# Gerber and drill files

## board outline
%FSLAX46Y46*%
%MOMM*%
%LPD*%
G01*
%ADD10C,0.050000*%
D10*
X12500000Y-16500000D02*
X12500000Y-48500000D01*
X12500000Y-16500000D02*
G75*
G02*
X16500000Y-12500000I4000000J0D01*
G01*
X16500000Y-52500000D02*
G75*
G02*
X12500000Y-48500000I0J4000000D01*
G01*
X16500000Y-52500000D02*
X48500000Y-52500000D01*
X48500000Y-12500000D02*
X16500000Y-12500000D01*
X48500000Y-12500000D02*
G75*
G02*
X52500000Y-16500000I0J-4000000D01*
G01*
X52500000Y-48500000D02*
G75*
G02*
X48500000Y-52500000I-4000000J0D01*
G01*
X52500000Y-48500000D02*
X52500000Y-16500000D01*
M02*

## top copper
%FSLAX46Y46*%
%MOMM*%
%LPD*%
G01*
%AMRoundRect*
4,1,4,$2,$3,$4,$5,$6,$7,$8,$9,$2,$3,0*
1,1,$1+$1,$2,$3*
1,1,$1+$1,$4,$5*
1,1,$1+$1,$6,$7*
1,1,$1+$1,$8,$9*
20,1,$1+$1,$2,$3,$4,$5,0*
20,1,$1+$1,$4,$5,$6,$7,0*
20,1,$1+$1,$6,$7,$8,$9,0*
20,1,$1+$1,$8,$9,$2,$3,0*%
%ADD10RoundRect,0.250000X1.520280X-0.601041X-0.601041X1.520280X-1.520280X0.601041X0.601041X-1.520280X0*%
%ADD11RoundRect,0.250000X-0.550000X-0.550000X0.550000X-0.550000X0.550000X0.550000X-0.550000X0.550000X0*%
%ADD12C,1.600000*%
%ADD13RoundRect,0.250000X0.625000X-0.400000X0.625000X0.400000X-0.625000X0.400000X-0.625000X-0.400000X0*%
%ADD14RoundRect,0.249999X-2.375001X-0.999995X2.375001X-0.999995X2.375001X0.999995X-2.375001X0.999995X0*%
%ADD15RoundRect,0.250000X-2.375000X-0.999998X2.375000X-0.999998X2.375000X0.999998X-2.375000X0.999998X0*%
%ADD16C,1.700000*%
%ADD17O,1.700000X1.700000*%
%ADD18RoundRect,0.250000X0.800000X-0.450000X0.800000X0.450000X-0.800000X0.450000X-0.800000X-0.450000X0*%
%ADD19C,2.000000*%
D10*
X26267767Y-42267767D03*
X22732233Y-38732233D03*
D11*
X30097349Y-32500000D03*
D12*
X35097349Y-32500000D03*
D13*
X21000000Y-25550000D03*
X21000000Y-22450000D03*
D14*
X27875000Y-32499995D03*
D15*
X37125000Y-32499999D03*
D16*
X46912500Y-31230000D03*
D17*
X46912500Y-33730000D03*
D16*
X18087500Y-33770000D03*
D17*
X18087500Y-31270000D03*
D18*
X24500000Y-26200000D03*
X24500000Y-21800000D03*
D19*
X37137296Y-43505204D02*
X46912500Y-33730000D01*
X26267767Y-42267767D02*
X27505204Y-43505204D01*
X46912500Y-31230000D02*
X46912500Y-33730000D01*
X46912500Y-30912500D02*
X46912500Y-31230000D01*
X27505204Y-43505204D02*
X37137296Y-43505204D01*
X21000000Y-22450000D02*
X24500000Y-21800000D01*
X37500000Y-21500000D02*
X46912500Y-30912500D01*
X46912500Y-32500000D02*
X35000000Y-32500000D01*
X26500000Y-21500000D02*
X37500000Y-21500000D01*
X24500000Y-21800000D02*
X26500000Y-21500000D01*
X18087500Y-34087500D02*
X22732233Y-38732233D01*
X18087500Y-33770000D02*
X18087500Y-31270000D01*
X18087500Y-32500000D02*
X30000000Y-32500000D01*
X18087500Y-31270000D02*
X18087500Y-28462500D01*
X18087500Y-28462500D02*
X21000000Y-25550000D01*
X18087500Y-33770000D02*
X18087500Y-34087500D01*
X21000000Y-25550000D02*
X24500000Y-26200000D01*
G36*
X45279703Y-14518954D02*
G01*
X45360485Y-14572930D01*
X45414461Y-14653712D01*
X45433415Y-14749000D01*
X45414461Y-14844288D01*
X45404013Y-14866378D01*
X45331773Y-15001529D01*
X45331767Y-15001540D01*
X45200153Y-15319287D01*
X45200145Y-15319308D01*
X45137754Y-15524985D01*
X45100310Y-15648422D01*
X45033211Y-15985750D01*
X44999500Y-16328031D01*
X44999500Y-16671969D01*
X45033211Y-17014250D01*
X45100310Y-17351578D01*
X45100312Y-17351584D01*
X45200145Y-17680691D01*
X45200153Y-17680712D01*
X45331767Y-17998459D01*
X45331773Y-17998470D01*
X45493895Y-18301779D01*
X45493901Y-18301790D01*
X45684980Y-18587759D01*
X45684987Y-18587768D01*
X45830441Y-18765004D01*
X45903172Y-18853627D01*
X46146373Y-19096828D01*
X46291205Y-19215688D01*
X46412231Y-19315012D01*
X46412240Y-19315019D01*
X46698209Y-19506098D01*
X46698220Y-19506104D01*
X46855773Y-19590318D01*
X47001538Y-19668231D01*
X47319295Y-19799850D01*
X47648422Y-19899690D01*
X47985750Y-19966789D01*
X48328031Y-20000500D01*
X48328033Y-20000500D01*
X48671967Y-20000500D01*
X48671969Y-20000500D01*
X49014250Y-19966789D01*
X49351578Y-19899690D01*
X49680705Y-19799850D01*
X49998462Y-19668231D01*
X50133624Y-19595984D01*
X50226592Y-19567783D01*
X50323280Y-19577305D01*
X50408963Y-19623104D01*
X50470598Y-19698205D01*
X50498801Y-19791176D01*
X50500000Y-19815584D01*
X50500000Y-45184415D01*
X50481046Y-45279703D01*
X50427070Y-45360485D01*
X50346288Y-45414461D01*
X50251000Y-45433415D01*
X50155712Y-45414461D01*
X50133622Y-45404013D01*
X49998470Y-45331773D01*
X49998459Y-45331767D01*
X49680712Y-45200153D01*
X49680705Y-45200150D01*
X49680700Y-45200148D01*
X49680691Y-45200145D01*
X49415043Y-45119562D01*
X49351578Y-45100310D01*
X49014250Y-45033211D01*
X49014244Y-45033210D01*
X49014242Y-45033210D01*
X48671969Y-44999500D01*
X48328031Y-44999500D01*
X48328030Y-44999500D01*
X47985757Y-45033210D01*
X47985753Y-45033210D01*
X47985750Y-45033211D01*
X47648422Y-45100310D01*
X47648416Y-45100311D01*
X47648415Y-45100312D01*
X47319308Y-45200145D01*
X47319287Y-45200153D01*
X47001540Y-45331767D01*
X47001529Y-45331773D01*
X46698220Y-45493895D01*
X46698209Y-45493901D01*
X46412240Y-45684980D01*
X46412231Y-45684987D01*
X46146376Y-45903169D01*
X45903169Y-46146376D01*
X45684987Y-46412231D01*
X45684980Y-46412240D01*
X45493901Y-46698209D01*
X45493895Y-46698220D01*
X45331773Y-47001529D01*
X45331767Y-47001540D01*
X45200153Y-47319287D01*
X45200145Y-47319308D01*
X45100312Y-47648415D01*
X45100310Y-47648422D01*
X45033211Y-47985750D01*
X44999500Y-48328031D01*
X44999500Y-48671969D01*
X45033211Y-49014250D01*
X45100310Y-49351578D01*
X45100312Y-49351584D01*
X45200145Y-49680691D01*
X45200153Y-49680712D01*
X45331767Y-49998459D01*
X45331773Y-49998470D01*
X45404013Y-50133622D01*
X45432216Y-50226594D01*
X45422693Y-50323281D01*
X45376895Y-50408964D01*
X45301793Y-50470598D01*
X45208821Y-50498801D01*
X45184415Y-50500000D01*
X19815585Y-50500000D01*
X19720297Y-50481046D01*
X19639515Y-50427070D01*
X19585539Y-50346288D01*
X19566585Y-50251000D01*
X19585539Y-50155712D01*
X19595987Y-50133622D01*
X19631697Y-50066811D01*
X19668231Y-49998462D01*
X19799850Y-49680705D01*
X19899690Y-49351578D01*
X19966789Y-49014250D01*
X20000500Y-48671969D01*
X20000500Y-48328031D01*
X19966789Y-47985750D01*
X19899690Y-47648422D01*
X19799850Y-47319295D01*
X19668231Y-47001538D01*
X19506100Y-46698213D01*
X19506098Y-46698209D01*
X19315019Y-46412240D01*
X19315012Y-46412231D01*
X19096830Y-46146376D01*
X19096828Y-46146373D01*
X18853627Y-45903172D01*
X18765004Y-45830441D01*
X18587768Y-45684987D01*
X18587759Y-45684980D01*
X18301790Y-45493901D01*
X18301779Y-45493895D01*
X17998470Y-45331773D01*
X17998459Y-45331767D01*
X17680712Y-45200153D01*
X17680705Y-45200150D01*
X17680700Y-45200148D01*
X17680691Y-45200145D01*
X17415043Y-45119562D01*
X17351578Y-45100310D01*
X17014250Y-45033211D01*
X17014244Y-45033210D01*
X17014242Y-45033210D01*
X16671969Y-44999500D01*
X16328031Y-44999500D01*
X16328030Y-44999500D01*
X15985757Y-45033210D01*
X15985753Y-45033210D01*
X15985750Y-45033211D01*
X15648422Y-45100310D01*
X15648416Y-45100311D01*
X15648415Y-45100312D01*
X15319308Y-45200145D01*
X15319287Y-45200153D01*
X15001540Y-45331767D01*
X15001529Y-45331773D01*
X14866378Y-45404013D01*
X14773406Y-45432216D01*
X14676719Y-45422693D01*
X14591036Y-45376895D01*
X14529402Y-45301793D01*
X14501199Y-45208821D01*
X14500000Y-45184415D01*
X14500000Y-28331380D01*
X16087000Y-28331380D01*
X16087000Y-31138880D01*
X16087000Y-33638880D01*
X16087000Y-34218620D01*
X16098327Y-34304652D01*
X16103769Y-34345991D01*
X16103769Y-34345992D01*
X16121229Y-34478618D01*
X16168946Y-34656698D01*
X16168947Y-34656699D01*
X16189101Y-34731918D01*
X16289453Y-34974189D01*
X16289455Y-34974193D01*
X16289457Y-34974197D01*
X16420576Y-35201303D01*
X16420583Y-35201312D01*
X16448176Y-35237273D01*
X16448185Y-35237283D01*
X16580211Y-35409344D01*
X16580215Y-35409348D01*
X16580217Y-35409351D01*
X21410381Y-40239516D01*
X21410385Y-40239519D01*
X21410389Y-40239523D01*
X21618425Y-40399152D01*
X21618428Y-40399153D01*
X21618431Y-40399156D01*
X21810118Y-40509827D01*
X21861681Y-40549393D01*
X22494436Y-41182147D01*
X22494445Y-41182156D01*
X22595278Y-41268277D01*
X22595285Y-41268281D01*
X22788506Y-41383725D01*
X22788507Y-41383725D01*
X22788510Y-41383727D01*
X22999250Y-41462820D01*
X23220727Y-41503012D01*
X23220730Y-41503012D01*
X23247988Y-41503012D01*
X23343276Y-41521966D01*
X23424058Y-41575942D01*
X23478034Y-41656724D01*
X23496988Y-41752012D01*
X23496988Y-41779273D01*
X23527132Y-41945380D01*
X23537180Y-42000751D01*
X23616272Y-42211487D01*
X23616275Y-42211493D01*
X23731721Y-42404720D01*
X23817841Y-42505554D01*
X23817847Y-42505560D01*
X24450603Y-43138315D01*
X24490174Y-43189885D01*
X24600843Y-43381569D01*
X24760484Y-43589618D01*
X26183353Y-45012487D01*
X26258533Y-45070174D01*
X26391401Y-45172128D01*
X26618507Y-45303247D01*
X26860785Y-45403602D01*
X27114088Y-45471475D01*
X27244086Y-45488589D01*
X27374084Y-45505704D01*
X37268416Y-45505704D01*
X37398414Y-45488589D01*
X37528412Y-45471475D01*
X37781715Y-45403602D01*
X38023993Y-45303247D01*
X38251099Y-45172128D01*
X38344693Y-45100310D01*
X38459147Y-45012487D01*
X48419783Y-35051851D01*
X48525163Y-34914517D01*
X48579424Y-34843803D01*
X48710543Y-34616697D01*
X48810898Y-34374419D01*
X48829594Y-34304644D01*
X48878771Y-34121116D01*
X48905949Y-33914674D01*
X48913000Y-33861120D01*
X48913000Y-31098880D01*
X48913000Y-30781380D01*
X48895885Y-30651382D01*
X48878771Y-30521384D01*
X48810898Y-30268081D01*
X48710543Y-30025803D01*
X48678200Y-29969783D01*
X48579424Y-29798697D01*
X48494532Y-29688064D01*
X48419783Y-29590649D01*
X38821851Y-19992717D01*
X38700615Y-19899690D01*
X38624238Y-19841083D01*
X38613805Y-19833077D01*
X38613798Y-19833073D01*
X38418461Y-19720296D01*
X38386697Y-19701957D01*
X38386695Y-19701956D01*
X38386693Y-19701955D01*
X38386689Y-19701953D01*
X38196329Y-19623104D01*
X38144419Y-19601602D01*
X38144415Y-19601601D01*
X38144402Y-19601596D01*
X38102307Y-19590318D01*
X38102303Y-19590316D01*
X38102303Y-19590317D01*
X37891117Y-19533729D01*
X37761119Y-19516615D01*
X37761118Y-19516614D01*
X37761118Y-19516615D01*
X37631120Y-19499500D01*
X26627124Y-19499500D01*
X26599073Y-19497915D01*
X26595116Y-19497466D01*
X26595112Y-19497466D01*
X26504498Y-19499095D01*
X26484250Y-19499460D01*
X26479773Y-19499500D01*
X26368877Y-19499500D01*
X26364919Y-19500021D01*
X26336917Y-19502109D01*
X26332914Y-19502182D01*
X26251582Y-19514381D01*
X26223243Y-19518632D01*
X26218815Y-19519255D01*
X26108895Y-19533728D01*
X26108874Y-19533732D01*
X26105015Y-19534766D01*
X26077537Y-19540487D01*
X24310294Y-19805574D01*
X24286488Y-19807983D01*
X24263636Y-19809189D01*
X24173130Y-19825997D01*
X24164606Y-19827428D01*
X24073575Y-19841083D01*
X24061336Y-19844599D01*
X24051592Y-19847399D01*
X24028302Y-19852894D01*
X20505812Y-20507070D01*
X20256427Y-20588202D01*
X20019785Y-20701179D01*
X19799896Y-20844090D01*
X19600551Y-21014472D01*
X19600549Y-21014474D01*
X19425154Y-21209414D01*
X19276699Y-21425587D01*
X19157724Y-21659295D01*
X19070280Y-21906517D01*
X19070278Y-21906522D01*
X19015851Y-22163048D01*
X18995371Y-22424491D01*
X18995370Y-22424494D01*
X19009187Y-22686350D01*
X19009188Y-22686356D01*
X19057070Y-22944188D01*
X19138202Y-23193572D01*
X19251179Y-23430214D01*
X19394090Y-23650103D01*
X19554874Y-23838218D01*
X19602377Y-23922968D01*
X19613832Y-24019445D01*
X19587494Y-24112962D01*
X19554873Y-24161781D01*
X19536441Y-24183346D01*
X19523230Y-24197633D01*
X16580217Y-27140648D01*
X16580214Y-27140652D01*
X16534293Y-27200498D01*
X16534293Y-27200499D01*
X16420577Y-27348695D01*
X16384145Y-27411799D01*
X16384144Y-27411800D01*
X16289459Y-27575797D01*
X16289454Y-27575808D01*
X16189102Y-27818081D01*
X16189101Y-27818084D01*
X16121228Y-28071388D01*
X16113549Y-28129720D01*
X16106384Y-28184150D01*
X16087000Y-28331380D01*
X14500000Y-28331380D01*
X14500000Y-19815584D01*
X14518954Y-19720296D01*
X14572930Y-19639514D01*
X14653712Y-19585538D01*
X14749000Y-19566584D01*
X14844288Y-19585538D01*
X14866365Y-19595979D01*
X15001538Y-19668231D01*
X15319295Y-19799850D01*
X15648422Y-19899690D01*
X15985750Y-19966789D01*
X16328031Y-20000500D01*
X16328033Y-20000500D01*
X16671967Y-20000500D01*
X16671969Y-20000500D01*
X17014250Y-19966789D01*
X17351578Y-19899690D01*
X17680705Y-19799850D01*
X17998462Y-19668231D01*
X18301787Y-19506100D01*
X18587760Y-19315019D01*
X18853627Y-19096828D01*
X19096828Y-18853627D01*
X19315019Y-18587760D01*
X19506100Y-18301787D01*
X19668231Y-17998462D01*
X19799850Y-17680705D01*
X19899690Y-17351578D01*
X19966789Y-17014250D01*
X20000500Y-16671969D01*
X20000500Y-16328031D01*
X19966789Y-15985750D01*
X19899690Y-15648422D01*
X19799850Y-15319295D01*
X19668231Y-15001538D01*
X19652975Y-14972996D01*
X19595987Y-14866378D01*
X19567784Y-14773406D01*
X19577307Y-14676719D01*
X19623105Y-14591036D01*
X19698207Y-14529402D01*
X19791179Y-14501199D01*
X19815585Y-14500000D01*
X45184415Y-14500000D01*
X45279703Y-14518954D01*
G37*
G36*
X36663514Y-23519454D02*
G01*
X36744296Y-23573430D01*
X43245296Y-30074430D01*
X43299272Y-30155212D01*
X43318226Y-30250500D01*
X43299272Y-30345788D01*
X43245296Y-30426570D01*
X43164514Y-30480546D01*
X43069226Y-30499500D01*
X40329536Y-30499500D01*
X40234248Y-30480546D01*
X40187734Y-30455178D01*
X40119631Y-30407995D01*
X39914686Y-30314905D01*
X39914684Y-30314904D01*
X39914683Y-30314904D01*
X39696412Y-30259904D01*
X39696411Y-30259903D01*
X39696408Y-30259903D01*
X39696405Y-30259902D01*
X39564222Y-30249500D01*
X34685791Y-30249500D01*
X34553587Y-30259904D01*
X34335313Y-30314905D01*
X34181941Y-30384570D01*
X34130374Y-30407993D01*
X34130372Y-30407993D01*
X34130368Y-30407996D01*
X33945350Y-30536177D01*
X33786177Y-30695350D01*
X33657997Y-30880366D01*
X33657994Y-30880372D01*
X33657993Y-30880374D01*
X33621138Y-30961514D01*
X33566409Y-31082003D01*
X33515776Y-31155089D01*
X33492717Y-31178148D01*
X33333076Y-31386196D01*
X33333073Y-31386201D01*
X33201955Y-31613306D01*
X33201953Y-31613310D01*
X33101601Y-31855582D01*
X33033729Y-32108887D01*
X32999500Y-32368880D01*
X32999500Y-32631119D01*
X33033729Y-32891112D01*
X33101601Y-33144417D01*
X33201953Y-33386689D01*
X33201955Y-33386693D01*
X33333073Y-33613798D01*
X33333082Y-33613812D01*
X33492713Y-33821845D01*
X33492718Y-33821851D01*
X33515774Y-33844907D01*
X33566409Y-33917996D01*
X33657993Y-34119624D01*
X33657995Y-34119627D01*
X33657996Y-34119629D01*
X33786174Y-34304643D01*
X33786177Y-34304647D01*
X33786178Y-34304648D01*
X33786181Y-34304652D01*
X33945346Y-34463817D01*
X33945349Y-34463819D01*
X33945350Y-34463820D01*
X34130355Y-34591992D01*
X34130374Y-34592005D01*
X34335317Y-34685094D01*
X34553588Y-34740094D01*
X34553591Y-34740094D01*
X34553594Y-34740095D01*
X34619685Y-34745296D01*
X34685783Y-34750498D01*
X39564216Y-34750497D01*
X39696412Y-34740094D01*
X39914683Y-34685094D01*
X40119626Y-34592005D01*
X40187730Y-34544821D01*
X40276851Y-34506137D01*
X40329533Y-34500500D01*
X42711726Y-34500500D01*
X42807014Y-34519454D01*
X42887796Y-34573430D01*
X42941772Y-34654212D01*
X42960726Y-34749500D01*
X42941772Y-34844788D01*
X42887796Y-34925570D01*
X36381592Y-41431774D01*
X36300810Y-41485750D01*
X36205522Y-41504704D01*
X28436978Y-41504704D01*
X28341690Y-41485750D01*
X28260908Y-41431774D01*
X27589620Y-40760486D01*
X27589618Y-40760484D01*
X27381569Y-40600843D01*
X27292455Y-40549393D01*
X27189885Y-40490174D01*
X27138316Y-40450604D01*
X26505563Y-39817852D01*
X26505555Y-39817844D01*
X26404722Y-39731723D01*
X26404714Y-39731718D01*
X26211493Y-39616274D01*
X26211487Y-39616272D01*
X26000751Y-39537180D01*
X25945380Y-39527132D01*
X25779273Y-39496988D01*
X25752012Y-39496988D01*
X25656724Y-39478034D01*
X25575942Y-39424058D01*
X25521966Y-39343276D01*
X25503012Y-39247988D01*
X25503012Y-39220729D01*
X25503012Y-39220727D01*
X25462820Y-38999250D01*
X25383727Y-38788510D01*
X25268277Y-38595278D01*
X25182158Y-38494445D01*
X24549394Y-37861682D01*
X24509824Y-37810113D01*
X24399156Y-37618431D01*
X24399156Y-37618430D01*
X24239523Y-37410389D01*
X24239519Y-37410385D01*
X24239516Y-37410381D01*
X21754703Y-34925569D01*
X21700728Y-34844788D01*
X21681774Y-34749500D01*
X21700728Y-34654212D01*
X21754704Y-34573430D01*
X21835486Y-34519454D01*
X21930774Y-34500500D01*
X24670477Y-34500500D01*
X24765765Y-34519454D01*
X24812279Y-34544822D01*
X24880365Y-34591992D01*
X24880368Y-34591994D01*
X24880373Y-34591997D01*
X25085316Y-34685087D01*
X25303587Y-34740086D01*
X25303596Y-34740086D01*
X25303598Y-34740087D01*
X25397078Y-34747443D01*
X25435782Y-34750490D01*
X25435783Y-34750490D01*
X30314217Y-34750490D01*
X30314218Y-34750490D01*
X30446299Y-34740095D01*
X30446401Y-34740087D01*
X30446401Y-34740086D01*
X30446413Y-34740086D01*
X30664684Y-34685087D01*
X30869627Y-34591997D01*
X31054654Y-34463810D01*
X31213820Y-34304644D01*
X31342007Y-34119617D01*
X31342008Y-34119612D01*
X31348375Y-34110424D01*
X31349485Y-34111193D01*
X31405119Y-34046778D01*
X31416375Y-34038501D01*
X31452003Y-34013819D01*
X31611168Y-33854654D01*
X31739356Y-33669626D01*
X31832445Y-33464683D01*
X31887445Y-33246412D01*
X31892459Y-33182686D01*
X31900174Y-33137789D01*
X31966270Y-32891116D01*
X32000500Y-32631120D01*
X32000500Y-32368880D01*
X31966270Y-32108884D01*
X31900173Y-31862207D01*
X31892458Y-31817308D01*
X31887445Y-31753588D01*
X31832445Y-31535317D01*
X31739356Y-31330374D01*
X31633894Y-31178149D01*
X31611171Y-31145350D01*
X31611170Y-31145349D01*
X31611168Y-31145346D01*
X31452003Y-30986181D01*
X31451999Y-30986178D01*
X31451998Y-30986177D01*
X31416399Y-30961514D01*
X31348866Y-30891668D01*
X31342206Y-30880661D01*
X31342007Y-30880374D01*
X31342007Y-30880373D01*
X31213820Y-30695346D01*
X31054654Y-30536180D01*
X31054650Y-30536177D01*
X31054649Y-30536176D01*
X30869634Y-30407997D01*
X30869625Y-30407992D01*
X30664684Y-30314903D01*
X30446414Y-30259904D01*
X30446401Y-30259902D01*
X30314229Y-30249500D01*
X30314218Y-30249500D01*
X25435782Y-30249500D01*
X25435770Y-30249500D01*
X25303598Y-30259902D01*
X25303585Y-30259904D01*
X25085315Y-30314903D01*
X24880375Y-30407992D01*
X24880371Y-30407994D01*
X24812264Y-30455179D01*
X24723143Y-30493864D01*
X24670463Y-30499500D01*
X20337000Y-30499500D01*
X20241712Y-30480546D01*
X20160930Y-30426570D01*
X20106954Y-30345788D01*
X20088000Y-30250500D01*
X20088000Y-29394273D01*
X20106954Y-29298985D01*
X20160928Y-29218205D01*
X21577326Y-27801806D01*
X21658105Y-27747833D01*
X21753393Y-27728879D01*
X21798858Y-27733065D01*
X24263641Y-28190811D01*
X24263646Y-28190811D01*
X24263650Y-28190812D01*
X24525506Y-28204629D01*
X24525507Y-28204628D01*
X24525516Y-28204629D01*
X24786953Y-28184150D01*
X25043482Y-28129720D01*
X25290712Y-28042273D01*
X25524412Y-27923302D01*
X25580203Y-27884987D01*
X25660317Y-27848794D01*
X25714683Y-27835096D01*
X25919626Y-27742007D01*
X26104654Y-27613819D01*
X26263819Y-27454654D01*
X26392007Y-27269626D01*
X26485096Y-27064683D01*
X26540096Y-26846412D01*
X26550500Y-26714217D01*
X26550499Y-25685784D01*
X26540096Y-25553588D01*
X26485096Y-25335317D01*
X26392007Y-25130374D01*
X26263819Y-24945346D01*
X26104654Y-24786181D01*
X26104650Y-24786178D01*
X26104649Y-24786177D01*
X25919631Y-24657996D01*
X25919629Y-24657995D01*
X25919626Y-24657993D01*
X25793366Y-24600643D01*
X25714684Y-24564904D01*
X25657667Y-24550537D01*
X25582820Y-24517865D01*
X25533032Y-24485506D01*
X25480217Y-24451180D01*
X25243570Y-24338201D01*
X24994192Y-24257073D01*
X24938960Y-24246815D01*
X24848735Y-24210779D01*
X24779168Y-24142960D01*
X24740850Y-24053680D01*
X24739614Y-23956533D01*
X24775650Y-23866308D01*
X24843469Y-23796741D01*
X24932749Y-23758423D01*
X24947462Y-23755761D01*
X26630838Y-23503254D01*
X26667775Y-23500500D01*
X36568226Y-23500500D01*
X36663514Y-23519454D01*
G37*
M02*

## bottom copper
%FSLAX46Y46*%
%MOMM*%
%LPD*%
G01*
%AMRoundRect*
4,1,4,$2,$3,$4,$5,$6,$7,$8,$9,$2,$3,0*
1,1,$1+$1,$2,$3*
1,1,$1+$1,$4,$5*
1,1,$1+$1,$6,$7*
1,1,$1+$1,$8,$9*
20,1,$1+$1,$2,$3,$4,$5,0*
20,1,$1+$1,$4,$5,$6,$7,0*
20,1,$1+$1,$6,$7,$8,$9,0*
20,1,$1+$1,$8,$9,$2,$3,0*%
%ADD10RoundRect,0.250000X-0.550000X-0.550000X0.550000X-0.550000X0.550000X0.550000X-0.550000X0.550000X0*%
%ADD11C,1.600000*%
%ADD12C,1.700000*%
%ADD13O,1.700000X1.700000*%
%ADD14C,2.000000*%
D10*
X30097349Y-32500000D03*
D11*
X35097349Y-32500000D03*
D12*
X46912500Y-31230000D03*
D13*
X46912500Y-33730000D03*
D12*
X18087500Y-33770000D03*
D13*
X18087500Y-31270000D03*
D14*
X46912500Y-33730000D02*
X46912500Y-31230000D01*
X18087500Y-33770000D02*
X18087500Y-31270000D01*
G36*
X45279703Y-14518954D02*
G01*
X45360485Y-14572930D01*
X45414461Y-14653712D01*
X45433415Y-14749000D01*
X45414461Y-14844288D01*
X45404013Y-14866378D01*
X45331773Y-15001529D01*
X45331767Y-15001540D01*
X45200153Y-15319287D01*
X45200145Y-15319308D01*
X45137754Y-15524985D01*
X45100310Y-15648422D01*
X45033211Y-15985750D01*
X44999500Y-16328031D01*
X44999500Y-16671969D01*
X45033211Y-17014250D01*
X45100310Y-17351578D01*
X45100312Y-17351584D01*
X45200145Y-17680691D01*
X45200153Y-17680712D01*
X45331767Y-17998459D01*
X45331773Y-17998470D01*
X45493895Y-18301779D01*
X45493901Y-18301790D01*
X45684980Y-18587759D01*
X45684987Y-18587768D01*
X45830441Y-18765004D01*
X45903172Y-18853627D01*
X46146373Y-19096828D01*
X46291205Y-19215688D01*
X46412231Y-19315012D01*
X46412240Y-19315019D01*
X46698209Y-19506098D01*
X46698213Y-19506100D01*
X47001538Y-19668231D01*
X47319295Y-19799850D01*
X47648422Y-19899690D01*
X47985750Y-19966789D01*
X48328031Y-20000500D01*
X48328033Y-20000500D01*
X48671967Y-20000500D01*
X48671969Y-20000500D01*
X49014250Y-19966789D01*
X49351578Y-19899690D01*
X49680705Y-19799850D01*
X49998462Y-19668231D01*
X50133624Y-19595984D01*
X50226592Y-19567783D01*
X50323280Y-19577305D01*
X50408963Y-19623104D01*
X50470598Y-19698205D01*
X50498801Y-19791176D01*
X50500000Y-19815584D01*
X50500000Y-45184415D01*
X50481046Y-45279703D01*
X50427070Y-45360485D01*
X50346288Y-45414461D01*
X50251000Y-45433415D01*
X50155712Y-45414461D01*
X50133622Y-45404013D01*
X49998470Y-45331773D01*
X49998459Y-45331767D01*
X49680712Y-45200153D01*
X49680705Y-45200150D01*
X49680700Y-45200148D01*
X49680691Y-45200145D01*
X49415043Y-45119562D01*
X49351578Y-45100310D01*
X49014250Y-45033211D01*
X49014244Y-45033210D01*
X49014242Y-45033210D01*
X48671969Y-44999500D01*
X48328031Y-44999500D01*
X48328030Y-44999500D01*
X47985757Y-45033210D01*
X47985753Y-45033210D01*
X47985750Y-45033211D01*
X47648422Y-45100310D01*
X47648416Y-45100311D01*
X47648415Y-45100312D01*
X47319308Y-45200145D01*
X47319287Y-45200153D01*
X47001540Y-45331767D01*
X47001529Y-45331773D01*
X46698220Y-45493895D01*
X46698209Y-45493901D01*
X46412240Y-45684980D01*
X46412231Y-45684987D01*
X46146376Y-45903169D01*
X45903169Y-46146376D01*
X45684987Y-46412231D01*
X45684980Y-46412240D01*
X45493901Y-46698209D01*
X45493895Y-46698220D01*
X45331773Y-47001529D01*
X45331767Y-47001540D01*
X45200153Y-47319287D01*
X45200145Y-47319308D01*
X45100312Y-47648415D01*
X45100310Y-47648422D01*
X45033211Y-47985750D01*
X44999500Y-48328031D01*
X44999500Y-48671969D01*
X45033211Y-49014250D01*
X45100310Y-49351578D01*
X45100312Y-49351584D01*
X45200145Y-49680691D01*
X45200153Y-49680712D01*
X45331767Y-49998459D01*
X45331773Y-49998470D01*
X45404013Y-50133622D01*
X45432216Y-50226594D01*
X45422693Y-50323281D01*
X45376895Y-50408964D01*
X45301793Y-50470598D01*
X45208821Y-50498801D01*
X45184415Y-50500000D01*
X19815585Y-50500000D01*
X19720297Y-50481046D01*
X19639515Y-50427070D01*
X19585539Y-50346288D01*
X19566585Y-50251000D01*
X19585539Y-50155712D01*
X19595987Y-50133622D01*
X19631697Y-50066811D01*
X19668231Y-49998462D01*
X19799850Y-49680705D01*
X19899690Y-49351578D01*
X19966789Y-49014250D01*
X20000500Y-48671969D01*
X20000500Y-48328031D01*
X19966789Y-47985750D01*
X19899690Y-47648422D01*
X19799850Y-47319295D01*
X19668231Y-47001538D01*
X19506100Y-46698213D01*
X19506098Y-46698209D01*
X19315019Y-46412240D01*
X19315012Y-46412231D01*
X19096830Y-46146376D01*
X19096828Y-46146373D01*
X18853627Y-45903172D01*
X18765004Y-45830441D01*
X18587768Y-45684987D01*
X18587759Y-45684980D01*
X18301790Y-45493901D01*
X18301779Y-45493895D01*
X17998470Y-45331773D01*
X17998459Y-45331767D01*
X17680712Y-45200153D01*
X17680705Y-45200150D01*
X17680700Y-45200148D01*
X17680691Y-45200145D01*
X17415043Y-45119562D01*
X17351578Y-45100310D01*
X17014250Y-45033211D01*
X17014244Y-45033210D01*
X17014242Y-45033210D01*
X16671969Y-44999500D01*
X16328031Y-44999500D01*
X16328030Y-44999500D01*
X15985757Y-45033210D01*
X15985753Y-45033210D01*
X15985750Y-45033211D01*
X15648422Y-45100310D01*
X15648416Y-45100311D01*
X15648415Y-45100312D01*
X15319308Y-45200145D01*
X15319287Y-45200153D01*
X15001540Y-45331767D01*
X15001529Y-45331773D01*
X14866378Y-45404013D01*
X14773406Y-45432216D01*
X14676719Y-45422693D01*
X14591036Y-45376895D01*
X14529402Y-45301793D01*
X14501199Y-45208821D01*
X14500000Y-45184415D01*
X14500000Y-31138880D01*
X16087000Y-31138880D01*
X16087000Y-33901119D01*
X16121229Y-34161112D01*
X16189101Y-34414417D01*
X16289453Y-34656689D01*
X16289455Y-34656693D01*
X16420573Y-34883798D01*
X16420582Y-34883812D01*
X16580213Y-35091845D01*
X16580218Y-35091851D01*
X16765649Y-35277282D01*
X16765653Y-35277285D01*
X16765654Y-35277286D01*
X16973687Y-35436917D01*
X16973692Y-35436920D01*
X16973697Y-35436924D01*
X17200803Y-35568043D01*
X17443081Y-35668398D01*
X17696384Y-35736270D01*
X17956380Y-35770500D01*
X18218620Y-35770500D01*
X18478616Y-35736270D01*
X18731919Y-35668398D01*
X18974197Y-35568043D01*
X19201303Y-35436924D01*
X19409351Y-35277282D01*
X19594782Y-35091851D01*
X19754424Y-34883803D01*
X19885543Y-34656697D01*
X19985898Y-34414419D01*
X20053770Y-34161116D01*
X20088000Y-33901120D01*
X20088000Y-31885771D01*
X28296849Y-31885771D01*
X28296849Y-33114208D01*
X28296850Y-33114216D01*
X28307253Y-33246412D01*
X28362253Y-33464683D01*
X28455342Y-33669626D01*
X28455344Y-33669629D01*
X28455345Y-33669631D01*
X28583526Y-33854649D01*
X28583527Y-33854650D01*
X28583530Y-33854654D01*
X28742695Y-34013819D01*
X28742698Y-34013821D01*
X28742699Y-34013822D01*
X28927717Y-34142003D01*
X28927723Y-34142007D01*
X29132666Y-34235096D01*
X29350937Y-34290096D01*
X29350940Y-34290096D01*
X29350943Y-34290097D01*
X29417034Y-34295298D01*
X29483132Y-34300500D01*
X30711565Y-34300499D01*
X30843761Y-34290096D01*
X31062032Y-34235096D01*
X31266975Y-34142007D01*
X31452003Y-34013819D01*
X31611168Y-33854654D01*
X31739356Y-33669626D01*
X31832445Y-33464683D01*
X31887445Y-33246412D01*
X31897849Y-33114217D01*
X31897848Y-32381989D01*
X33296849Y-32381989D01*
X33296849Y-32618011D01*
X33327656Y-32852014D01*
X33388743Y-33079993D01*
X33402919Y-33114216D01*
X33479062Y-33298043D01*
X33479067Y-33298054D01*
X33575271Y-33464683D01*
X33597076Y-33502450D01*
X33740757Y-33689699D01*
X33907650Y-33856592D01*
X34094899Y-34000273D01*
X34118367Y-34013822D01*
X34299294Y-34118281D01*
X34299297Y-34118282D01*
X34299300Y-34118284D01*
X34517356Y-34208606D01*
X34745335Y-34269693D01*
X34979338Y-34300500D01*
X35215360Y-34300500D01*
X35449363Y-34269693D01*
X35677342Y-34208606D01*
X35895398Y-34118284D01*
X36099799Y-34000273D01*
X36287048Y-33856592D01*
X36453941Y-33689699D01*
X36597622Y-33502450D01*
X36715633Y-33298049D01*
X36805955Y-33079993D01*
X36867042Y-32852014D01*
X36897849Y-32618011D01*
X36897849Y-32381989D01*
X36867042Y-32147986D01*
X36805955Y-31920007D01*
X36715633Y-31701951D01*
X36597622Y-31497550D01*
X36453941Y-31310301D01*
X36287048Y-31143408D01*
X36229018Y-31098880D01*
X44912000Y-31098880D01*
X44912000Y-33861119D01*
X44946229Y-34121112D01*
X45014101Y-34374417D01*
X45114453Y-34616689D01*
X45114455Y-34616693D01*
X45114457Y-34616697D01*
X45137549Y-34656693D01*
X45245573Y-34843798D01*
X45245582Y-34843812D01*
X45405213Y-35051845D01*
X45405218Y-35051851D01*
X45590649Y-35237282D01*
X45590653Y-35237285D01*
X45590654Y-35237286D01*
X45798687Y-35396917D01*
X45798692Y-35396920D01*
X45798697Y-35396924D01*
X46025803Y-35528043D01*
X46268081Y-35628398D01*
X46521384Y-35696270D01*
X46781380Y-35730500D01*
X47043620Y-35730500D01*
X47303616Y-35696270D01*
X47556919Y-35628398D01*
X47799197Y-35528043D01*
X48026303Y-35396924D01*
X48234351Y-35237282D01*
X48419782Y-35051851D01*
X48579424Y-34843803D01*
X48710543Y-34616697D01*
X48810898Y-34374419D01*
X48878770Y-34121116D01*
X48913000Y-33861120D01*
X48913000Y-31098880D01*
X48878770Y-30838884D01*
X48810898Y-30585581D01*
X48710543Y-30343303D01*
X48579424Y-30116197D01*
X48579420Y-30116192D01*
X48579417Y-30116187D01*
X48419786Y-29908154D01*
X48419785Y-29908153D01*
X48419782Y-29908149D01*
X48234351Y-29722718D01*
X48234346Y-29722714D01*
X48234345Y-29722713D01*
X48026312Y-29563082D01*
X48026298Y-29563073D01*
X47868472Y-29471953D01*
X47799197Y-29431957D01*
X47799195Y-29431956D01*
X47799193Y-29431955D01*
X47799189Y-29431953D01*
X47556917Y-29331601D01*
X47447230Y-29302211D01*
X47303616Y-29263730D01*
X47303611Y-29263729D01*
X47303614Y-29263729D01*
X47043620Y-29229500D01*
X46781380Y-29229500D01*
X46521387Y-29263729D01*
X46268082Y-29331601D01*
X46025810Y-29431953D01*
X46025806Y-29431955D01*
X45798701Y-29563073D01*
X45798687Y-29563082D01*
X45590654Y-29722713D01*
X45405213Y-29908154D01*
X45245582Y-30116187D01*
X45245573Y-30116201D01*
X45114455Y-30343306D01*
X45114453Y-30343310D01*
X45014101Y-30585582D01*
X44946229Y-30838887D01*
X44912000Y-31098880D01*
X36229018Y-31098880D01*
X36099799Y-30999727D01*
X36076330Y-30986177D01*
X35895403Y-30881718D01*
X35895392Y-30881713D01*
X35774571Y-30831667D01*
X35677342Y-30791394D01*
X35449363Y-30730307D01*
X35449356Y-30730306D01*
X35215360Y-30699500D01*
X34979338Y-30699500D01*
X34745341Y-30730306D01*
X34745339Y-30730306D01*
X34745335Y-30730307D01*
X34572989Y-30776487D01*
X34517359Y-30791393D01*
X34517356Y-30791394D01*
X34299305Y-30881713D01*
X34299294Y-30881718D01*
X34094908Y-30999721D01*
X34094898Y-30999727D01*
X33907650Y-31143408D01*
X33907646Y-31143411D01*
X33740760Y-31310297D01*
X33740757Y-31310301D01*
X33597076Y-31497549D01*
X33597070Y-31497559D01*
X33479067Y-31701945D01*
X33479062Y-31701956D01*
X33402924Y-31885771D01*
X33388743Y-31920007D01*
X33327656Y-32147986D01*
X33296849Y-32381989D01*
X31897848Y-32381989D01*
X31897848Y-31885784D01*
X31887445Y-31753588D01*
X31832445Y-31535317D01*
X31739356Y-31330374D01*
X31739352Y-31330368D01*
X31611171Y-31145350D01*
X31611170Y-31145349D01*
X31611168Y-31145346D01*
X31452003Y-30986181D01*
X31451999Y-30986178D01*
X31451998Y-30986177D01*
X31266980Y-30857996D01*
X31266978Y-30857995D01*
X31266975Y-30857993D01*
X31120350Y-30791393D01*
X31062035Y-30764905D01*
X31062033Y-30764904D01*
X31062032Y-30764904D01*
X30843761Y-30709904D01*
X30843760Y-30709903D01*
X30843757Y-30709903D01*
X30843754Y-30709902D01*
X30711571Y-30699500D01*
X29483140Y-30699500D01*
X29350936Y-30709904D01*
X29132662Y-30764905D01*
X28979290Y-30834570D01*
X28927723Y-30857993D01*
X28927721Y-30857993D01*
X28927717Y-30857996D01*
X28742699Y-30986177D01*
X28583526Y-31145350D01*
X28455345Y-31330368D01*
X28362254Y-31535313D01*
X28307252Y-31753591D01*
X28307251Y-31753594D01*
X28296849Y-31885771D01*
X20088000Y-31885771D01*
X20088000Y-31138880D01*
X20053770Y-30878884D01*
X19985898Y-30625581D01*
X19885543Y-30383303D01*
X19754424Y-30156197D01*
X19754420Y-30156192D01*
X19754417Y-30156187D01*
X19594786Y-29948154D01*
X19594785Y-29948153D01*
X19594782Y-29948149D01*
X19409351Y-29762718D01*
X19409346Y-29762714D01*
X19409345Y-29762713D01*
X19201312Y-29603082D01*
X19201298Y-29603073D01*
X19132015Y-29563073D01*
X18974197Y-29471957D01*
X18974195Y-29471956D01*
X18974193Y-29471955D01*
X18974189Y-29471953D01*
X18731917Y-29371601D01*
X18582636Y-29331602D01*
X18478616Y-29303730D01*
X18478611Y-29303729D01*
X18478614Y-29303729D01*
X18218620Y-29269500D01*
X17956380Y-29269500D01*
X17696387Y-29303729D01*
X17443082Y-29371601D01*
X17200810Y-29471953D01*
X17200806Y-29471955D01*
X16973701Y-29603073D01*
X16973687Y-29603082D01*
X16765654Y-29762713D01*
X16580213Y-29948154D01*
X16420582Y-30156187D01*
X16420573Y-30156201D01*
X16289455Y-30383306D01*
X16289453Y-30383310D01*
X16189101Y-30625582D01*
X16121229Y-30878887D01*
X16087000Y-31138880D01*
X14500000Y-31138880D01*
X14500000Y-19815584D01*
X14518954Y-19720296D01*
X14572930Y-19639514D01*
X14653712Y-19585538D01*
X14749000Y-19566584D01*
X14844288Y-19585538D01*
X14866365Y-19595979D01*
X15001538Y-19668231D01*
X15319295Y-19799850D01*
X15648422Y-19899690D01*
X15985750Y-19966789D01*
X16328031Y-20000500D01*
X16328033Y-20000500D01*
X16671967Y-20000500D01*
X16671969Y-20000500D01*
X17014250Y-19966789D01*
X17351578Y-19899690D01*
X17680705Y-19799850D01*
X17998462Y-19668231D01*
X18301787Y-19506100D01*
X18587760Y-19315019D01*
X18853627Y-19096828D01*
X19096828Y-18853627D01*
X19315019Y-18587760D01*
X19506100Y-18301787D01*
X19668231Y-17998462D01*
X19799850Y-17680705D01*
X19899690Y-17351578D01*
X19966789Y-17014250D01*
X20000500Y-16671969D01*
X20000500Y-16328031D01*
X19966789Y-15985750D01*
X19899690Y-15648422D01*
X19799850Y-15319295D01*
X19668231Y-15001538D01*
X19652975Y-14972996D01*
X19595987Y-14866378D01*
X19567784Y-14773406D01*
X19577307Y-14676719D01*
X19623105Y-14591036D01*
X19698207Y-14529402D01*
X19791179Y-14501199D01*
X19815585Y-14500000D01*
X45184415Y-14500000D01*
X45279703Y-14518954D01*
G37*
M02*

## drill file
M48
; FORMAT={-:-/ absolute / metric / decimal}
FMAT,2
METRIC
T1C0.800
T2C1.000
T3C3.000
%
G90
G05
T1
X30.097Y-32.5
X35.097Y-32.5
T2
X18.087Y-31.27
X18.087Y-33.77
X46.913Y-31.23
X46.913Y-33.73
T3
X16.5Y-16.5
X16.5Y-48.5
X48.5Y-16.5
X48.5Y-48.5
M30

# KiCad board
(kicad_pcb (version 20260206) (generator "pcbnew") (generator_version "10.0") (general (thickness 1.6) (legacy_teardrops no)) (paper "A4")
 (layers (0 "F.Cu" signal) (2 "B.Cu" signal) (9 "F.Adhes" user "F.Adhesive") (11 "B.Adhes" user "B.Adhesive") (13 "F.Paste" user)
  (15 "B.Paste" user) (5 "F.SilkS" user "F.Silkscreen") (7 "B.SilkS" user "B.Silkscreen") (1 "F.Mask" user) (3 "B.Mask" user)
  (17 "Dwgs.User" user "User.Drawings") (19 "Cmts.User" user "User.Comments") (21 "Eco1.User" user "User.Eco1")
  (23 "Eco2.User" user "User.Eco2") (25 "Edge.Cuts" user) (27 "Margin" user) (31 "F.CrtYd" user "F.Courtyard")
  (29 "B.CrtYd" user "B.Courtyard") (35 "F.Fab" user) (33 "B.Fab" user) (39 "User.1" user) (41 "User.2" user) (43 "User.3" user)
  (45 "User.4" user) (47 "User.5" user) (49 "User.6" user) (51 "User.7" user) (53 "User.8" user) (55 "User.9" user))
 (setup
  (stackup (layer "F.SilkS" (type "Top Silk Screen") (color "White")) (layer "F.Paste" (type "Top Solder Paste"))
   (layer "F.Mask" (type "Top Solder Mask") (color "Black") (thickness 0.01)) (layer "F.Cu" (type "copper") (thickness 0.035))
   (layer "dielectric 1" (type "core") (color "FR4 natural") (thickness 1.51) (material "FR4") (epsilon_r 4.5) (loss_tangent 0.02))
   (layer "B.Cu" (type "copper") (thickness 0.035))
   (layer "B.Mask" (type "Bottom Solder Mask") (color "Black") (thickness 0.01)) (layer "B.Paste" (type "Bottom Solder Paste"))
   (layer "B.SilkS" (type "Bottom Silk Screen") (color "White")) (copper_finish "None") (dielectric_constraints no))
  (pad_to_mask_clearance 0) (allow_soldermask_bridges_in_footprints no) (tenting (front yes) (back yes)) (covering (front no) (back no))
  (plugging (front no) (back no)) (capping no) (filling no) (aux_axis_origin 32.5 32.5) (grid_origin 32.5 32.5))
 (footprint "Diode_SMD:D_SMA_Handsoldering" (layer "F.Cu") (at 24.5 40.5 135)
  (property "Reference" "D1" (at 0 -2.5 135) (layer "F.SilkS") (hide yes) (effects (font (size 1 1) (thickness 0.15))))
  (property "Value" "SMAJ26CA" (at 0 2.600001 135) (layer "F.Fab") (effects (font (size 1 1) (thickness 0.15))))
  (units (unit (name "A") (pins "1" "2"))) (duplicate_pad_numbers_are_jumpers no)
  (pad "1" smd roundrect (at -2.5 0 135) (size 3.5 1.8) (layers "F.Cu" "F.Mask" "F.Paste") (roundrect_rratio 0.1388888889)
   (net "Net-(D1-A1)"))
  (pad "2" smd roundrect (at 2.5 0 135) (size 3.5 1.8) (layers "F.Cu" "F.Mask" "F.Paste") (roundrect_rratio 0.1388888889)
   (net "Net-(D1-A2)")))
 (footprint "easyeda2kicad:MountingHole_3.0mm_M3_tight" (layer "F.Cu") (at 16.5 16.5 90)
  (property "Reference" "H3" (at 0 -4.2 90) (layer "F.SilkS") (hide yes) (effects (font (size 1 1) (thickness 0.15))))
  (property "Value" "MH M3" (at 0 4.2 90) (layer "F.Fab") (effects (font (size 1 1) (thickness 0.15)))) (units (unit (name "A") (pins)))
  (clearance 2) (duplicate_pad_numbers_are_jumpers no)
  (pad "" np_thru_hole circle (at 0 0 90) (size 3 3) (drill 3) (layers "*.Cu" "*.Mask")))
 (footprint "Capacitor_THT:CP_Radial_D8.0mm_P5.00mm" (layer "F.Cu") (at 30.097349 32.5)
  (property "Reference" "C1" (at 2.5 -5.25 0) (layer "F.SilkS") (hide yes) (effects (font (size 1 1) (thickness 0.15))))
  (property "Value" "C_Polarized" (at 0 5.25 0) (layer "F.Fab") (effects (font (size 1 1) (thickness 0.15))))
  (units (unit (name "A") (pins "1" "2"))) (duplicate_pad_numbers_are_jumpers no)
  (pad "1" thru_hole roundrect (at 0 0) (size 1.6 1.6) (drill 0.8) (layers "*.Cu" "*.Mask") (remove_unused_layers no)
   (roundrect_rratio 0.15625) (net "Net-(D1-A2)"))
  (pad "2" thru_hole circle (at 5 0) (size 1.6 1.6) (drill 0.8) (layers "*.Cu" "*.Mask") (remove_unused_layers no) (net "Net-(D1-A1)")))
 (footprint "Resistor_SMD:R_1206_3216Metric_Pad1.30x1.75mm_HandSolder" (layer "F.Cu") (at 21 24 90)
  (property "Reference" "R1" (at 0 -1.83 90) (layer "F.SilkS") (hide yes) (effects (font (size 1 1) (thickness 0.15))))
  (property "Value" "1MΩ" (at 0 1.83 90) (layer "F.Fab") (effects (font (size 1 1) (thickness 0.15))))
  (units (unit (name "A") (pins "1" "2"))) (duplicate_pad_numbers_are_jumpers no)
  (pad "1" smd roundrect (at -1.55 0 90) (size 1.3 1.75) (layers "F.Cu" "F.Mask" "F.Paste") (roundrect_rratio 0.192308) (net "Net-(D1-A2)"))
  (pad "2" smd roundrect (at 1.55 0 90) (size 1.3 1.75) (layers "F.Cu" "F.Mask" "F.Paste") (roundrect_rratio 0.192308) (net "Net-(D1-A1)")))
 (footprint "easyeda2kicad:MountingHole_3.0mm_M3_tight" (layer "F.Cu") (at 16.5 48.5 90)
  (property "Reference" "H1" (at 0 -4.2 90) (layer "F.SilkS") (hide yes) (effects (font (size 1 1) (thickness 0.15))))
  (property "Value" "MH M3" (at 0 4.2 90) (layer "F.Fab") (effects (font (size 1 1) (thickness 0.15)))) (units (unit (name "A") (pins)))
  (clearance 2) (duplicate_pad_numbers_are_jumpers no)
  (pad "" np_thru_hole circle (at 0 0 90) (size 3 3) (drill 3) (layers "*.Cu" "*.Mask")))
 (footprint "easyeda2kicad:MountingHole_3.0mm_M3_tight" (layer "F.Cu") (at 48.5 16.5 90)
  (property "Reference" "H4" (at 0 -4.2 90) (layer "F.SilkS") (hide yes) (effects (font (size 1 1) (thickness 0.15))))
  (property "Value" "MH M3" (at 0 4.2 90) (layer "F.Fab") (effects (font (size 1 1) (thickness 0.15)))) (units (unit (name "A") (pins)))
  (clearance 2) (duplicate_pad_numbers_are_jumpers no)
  (pad "" np_thru_hole circle (at 0 0 90) (size 3 3) (drill 3) (layers "*.Cu" "*.Mask")))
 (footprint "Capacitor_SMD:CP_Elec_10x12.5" (layer "F.Cu") (at 32.5 32.5)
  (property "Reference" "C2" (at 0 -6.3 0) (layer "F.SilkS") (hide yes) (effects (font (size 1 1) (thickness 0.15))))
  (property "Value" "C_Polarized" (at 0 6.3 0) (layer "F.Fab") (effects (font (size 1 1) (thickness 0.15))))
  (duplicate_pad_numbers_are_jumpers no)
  (pad "1" smd roundrect (at -4.625 -0.000005) (size 5.25 2.499989) (layers "F.Cu" "F.Mask" "F.Paste") (roundrect_rratio 0.1)
   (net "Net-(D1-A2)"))
  (pad "2" smd roundrect (at 4.625 -0.000001) (size 5.25 2.499997) (layers "F.Cu" "F.Mask" "F.Paste") (roundrect_rratio 0.1)
   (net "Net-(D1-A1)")))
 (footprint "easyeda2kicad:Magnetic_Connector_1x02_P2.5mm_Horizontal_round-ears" (layer "F.Cu") (at 47.0125 32.5)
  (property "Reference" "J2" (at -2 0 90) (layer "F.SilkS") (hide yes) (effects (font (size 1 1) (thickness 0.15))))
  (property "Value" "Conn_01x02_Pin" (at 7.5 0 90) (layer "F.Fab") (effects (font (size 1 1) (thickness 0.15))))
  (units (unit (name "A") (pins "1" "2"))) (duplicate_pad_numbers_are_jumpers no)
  (pad "1" thru_hole circle (at -0.1 -1.27) (size 1.7 1.7) (drill 1) (layers "*.Cu" "*.Mask") (remove_unused_layers no) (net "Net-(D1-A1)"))
  (pad "2" thru_hole oval (at -0.1 1.23) (size 1.7 1.7) (drill 1) (layers "*.Cu" "*.Mask") (remove_unused_layers no) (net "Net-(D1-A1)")))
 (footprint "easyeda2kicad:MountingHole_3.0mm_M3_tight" (layer "F.Cu") (at 48.5 48.5 90)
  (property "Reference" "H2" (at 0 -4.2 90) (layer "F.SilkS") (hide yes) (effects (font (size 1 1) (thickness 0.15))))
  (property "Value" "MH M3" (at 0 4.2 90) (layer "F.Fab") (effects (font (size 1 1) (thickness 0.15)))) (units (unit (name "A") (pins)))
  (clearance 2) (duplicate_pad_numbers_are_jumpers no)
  (pad "" np_thru_hole circle (at 0 0 90) (size 3 3) (drill 3) (layers "*.Cu" "*.Mask")))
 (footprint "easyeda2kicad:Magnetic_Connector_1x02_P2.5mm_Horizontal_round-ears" (layer "F.Cu") (at 17.9875 32.5 180)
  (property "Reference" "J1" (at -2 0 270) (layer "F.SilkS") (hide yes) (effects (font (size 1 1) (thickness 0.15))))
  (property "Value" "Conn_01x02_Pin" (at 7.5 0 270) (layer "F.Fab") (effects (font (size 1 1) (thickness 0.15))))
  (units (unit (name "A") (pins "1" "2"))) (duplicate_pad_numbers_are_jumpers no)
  (pad "1" thru_hole circle (at -0.1 -1.27 180) (size 1.7 1.7) (drill 1) (layers "*.Cu" "*.Mask") (remove_unused_layers no)
   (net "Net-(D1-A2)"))
  (pad "2" thru_hole oval (at -0.1 1.23 180) (size 1.7 1.7) (drill 1) (layers "*.Cu" "*.Mask") (remove_unused_layers no) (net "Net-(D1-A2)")))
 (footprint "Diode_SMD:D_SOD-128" (layer "F.Cu") (at 24.5 24 90)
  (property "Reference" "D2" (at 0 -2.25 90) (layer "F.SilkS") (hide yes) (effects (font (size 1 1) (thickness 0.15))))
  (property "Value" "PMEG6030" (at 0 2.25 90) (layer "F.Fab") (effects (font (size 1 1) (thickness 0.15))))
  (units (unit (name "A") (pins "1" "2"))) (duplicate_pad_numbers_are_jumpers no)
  (pad "1" smd roundrect (at -2.2 0 90) (size 1.4 2.1) (layers "F.Cu" "F.Mask" "F.Paste") (roundrect_rratio 0.1785714286)
   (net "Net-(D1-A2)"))
  (pad "2" smd roundrect (at 2.2 0 90) (size 1.4 2.1) (layers "F.Cu" "F.Mask" "F.Paste") (roundrect_rratio 0.1785714286) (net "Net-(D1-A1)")))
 (gr_line (start 12.5 16.5) (end 12.5 48.5) (stroke (width 0.05) (type default)) (layer "Edge.Cuts"))
 (gr_arc (start 12.5 16.5) (mid 13.671573 13.671573) (end 16.5 12.5) (stroke (width 0.05) (type default)) (layer "Edge.Cuts"))
 (gr_arc (start 16.5 52.5) (mid 13.671573 51.328427) (end 12.5 48.5) (stroke (width 0.05) (type default)) (layer "Edge.Cuts"))
 (gr_line (start 16.5 52.5) (end 48.5 52.5) (stroke (width 0.05) (type default)) (layer "Edge.Cuts"))
 (gr_line (start 48.5 12.5) (end 16.5 12.5) (stroke (width 0.05) (type default)) (layer "Edge.Cuts"))
 (gr_arc (start 48.5 12.5) (mid 51.328427 13.671573) (end 52.5 16.5) (stroke (width 0.05) (type default)) (layer "Edge.Cuts"))
 (gr_arc (start 52.5 48.5) (mid 51.328427 51.328427) (end 48.5 52.5) (stroke (width 0.05) (type default)) (layer "Edge.Cuts"))
 (gr_line (start 52.5 48.5) (end 52.5 16.5) (stroke (width 0.05) (type default)) (layer "Edge.Cuts"))
 (segment (start 37.137296 43.505204) (end 46.9125 33.73) (width 2) (layer "F.Cu") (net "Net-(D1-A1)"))
 (segment (start 26.267767 42.267767) (end 27.505204 43.505204) (width 2) (layer "F.Cu") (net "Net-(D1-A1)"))
 (segment (start 46.9125 31.23) (end 46.9125 33.73) (width 2) (layer "F.Cu") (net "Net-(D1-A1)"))
 (segment (start 46.9125 30.9125) (end 46.9125 31.23) (width 2) (layer "F.Cu") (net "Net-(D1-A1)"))
 (segment (start 27.505204 43.505204) (end 37.137296 43.505204) (width 2) (layer "F.Cu") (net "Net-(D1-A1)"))
 (segment (start 21 22.45) (end 24.5 21.8) (width 2) (layer "F.Cu") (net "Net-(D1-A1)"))
 (segment (start 37.5 21.5) (end 46.9125 30.9125) (width 2) (layer "F.Cu") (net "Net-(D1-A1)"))
 (segment (start 46.9125 32.5) (end 35 32.5) (width 2) (layer "F.Cu") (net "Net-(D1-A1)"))
 (segment (start 26.5 21.5) (end 37.5 21.5) (width 2) (layer "F.Cu") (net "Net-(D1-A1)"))
 (segment (start 24.5 21.8) (end 26.5 21.5) (width 2) (layer "F.Cu") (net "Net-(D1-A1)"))
 (segment (start 46.9125 33.73) (end 46.9125 31.23) (width 2) (layer "B.Cu") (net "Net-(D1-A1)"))
 (segment (start 18.0875 34.0875) (end 22.732233 38.732233) (width 2) (layer "F.Cu") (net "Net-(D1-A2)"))
 (segment (start 18.0875 33.77) (end 18.0875 31.27) (width 2) (layer "F.Cu") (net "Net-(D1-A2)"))
 (segment (start 18.0875 32.5) (end 30 32.5) (width 2) (layer "F.Cu") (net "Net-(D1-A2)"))
 (segment (start 18.0875 31.27) (end 18.0875 28.4625) (width 2) (layer "F.Cu") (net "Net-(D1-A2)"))
 (segment (start 18.0875 28.4625) (end 21 25.55) (width 2) (layer "F.Cu") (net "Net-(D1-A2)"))
 (segment (start 18.0875 33.77) (end 18.0875 34.0875) (width 2) (layer "F.Cu") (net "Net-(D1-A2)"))
 (segment (start 21 25.55) (end 24.5 26.2) (width 2) (layer "F.Cu") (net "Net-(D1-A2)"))
 (segment (start 18.0875 33.77) (end 18.0875 31.27) (width 2) (layer "B.Cu") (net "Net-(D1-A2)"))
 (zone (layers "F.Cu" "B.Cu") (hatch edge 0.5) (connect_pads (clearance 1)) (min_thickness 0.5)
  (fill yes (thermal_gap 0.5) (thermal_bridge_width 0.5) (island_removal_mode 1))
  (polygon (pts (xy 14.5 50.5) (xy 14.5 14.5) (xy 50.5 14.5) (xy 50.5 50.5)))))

